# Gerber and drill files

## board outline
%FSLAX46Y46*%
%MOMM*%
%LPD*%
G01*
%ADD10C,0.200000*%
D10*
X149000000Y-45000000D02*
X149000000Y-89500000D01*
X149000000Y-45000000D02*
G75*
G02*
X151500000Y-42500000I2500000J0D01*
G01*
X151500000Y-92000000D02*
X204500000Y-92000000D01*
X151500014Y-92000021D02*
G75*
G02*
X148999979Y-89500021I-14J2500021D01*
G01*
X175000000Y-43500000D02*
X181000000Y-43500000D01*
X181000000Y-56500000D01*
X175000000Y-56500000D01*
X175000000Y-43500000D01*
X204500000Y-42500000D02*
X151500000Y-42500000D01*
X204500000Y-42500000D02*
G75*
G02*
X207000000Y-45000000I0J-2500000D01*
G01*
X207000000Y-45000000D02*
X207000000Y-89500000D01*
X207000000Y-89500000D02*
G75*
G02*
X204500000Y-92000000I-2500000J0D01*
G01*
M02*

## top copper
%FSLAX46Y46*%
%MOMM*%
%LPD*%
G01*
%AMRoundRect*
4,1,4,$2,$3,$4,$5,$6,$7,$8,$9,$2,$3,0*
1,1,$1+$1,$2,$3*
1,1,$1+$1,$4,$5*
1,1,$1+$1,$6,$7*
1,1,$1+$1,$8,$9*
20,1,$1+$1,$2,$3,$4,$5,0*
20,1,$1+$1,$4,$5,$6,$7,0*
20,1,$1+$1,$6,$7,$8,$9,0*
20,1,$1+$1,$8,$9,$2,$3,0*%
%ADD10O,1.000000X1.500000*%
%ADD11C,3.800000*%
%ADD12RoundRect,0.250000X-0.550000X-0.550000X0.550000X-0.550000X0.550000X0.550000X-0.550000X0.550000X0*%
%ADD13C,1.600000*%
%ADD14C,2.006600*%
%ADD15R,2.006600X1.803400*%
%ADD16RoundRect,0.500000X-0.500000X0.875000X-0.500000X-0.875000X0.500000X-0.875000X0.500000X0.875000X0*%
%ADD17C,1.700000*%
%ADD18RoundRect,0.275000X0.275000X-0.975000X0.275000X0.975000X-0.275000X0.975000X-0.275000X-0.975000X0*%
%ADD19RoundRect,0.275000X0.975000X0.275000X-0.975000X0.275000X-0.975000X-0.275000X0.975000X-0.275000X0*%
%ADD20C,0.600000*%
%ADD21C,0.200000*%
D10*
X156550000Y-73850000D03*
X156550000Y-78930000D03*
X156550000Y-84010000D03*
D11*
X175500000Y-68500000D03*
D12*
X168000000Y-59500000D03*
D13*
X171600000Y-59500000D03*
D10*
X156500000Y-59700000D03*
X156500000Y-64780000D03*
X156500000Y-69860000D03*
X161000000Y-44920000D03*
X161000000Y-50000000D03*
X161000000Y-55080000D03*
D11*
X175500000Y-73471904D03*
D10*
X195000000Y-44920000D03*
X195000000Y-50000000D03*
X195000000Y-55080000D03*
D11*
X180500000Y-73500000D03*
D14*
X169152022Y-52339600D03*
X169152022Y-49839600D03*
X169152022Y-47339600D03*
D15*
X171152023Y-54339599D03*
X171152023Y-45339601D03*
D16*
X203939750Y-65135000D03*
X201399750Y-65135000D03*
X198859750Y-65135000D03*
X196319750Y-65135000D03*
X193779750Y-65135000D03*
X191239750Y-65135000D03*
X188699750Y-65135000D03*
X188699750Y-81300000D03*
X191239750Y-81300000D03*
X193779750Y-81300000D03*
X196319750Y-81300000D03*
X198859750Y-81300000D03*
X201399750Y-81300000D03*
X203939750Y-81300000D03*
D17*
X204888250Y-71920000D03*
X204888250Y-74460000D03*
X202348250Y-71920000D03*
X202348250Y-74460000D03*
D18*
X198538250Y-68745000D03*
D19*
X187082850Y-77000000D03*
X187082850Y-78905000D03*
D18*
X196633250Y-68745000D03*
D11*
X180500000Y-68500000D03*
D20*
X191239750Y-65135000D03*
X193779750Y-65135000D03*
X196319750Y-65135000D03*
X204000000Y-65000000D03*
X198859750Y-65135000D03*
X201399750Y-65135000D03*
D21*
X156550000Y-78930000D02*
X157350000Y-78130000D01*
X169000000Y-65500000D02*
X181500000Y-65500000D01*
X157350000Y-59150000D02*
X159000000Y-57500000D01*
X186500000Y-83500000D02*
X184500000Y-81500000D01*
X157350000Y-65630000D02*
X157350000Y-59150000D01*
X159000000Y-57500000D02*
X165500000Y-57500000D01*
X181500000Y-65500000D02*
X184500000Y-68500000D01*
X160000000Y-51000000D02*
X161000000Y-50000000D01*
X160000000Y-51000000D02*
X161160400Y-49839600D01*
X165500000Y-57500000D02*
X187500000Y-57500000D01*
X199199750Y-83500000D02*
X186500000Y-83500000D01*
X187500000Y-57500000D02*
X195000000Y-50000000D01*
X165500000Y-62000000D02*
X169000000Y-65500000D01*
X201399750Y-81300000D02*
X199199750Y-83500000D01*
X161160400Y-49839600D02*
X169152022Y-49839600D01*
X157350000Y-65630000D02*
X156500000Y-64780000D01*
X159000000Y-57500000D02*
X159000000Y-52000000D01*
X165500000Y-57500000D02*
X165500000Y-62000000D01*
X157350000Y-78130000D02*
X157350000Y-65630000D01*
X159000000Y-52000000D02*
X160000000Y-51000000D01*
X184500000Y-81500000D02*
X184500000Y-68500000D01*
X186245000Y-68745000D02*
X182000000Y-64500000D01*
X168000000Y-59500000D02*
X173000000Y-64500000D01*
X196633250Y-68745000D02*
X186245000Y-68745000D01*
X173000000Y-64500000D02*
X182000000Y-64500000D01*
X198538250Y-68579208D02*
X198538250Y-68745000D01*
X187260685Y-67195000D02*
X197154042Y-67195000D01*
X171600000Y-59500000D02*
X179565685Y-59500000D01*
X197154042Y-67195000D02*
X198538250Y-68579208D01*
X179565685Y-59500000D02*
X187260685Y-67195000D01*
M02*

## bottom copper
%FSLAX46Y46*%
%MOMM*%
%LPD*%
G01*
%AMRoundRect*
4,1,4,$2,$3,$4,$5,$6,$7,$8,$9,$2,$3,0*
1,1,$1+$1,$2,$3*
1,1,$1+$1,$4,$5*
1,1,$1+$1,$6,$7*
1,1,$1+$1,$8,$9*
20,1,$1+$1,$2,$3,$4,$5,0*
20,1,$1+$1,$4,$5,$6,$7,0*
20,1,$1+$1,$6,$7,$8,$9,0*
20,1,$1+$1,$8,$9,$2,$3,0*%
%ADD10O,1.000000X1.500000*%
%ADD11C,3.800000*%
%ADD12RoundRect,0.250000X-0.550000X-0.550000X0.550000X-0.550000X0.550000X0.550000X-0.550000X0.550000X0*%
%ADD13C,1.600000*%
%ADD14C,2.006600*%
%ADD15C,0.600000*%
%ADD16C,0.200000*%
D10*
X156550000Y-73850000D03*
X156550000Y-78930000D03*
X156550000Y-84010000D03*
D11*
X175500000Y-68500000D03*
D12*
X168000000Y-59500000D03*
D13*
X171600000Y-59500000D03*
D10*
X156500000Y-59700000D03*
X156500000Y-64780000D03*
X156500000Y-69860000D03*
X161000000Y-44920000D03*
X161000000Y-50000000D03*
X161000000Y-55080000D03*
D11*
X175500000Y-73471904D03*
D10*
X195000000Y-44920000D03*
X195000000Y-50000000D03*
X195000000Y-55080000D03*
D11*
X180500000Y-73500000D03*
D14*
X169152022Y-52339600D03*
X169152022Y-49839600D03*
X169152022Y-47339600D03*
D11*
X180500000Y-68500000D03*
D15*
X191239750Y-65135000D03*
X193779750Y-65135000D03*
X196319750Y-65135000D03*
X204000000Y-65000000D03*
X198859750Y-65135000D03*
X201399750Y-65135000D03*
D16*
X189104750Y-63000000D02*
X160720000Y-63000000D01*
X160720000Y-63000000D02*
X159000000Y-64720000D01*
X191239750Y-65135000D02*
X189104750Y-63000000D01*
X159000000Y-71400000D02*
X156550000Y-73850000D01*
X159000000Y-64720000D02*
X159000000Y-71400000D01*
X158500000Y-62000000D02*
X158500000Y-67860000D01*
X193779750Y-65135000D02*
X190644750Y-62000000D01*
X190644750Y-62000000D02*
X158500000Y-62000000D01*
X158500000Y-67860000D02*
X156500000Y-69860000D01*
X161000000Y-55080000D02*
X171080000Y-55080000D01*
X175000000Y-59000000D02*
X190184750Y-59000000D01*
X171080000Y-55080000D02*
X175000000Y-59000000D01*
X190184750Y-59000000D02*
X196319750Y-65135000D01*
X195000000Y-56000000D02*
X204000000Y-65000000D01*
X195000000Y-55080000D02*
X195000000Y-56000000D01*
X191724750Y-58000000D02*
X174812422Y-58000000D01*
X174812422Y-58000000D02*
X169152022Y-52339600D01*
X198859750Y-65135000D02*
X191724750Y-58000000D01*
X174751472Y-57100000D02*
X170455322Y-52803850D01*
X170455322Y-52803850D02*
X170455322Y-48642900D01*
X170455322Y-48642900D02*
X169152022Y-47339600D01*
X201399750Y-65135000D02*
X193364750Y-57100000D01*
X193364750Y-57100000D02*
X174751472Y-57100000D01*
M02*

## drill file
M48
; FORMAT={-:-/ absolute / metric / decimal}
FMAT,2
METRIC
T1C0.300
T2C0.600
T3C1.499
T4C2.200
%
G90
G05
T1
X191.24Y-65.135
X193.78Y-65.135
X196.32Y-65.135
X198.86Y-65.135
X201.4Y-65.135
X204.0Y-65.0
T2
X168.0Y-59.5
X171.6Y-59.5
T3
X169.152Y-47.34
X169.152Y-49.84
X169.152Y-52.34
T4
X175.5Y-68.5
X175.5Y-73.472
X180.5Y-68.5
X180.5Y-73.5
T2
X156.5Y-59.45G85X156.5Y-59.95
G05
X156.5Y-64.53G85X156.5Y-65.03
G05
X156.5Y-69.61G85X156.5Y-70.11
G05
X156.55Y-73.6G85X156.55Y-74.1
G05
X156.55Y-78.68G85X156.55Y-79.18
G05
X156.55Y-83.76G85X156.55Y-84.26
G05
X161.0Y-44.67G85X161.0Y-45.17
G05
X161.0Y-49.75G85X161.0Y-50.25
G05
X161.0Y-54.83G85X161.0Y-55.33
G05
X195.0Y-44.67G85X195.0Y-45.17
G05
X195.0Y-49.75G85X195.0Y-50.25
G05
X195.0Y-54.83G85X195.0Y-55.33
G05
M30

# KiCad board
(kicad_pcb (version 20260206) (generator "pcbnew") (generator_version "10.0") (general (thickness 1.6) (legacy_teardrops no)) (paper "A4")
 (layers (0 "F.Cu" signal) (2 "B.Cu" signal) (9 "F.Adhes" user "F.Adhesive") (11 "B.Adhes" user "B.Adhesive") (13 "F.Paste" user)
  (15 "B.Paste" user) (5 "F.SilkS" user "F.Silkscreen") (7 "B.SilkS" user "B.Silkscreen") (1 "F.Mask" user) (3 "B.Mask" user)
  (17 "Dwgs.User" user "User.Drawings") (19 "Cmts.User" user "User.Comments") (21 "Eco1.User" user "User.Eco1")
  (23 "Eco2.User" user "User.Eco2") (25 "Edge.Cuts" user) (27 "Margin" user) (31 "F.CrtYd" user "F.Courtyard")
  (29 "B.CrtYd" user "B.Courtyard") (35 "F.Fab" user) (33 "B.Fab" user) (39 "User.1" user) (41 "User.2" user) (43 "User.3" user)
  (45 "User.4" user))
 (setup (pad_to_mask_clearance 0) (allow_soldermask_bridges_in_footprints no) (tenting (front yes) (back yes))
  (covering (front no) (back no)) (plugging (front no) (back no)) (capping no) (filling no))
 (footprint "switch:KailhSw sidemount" (layer "F.Cu") (at 156.55 73.85 -90)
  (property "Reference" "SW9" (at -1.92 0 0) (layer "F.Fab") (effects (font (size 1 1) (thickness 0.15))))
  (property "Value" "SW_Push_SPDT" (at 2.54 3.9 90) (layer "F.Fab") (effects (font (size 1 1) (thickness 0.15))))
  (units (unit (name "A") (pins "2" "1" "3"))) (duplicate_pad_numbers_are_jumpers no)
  (pad "1" thru_hole oval (at 0 0 270) (size 1.5 1) (drill oval 1.1 0.6) (layers "*.Cu" "*.Mask") (remove_unused_layers no) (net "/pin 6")
   (thermal_bridge_angle 45))
  (pad "2" thru_hole oval (at 5.08 0 270) (size 1.5 1) (drill oval 1.1 0.6) (layers "*.Cu" "*.Mask") (remove_unused_layers no)
   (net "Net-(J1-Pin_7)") (thermal_bridge_angle 45))
  (pad "3" thru_hole oval (at 10.16 0 270) (size 1.5 1) (drill oval 1.1 0.6) (layers "*.Cu" "*.Mask") (remove_unused_layers no)
   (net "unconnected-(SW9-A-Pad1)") (thermal_bridge_angle 45)))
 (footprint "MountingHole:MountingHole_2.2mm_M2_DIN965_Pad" (layer "F.Cu") (at 175.5 68.5)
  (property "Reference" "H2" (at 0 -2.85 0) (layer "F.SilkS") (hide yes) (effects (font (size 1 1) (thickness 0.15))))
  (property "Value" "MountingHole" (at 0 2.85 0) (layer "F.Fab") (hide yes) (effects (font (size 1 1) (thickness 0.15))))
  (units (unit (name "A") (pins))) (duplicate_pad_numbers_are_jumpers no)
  (pad "1" thru_hole circle (at 0 0) (size 3.8 3.8) (drill 2.2) (layers "*.Cu" "*.Mask") (remove_unused_layers no) (zone_connect 2)))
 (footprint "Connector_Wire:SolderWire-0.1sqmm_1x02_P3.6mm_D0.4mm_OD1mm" (layer "F.Cu") (at 168 59.5)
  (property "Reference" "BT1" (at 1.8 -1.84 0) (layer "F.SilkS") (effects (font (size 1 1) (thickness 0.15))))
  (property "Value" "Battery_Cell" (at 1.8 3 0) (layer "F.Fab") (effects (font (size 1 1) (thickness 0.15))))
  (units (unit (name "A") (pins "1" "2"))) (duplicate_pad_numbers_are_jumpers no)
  (pad "1" thru_hole roundrect (at 0 0) (size 1.6 1.6) (drill 0.6) (layers "*.Cu" "*.Mask") (remove_unused_layers no)
   (roundrect_rratio 0.15625) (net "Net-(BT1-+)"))
  (pad "2" thru_hole circle (at 3.6 0) (size 1.6 1.6) (drill 0.6) (layers "*.Cu" "*.Mask") (remove_unused_layers no) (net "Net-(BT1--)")))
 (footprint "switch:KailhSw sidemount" (layer "F.Cu") (at 156.5 59.7 -90)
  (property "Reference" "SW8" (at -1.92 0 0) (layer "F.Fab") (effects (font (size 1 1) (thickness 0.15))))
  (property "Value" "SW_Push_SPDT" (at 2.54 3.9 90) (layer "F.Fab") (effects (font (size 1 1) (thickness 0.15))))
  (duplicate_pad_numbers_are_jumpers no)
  (pad "1" thru_hole oval (at 0 0 270) (size 1.5 1) (drill oval 1.1 0.6) (layers "*.Cu" "*.Mask") (remove_unused_layers no)
   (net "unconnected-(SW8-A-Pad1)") (thermal_bridge_angle 45))
  (pad "2" thru_hole oval (at 5.08 0 270) (size 1.5 1) (drill oval 1.1 0.6) (layers "*.Cu" "*.Mask") (remove_unused_layers no)
   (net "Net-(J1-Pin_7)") (thermal_bridge_angle 45))
  (pad "3" thru_hole oval (at 10.16 0 270) (size 1.5 1) (drill oval 1.1 0.6) (layers "*.Cu" "*.Mask") (remove_unused_layers no)
   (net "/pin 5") (thermal_bridge_angle 45)))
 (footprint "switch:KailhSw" (layer "F.Cu") (at 161 44.92 -90)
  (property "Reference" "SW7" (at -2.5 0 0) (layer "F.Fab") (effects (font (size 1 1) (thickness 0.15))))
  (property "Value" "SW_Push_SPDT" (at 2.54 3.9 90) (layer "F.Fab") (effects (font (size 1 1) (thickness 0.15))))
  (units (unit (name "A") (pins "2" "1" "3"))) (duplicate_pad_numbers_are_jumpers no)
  (pad "1" thru_hole oval (at 0 0 270) (size 1.5 1) (drill oval 1.1 0.6) (layers "*.Cu" "*.Mask") (remove_unused_layers no)
   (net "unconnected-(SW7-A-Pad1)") (thermal_bridge_angle 45))
  (pad "2" thru_hole oval (at 5.08 0 270) (size 1.5 1) (drill oval 1.1 0.6) (layers "*.Cu" "*.Mask") (remove_unused_layers no)
   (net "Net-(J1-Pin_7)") (thermal_bridge_angle 45))
  (pad "3" thru_hole oval (at 10.16 0 270) (size 1.5 1) (drill oval 1.1 0.6) (layers "*.Cu" "*.Mask") (remove_unused_layers no)
   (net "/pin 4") (thermal_bridge_angle 45)))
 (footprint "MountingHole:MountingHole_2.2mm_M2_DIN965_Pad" (layer "F.Cu") (at 175.5 73.471904)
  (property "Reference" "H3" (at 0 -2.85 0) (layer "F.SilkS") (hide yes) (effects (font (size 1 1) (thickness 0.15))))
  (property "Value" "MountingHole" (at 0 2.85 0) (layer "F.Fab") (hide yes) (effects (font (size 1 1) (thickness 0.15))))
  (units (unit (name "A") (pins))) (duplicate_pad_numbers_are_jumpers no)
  (pad "1" thru_hole circle (at 0 0) (size 3.8 3.8) (drill 2.2) (layers "*.Cu" "*.Mask") (remove_unused_layers no) (zone_connect 2)))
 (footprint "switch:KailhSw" (layer "F.Cu") (at 195 44.92 -90)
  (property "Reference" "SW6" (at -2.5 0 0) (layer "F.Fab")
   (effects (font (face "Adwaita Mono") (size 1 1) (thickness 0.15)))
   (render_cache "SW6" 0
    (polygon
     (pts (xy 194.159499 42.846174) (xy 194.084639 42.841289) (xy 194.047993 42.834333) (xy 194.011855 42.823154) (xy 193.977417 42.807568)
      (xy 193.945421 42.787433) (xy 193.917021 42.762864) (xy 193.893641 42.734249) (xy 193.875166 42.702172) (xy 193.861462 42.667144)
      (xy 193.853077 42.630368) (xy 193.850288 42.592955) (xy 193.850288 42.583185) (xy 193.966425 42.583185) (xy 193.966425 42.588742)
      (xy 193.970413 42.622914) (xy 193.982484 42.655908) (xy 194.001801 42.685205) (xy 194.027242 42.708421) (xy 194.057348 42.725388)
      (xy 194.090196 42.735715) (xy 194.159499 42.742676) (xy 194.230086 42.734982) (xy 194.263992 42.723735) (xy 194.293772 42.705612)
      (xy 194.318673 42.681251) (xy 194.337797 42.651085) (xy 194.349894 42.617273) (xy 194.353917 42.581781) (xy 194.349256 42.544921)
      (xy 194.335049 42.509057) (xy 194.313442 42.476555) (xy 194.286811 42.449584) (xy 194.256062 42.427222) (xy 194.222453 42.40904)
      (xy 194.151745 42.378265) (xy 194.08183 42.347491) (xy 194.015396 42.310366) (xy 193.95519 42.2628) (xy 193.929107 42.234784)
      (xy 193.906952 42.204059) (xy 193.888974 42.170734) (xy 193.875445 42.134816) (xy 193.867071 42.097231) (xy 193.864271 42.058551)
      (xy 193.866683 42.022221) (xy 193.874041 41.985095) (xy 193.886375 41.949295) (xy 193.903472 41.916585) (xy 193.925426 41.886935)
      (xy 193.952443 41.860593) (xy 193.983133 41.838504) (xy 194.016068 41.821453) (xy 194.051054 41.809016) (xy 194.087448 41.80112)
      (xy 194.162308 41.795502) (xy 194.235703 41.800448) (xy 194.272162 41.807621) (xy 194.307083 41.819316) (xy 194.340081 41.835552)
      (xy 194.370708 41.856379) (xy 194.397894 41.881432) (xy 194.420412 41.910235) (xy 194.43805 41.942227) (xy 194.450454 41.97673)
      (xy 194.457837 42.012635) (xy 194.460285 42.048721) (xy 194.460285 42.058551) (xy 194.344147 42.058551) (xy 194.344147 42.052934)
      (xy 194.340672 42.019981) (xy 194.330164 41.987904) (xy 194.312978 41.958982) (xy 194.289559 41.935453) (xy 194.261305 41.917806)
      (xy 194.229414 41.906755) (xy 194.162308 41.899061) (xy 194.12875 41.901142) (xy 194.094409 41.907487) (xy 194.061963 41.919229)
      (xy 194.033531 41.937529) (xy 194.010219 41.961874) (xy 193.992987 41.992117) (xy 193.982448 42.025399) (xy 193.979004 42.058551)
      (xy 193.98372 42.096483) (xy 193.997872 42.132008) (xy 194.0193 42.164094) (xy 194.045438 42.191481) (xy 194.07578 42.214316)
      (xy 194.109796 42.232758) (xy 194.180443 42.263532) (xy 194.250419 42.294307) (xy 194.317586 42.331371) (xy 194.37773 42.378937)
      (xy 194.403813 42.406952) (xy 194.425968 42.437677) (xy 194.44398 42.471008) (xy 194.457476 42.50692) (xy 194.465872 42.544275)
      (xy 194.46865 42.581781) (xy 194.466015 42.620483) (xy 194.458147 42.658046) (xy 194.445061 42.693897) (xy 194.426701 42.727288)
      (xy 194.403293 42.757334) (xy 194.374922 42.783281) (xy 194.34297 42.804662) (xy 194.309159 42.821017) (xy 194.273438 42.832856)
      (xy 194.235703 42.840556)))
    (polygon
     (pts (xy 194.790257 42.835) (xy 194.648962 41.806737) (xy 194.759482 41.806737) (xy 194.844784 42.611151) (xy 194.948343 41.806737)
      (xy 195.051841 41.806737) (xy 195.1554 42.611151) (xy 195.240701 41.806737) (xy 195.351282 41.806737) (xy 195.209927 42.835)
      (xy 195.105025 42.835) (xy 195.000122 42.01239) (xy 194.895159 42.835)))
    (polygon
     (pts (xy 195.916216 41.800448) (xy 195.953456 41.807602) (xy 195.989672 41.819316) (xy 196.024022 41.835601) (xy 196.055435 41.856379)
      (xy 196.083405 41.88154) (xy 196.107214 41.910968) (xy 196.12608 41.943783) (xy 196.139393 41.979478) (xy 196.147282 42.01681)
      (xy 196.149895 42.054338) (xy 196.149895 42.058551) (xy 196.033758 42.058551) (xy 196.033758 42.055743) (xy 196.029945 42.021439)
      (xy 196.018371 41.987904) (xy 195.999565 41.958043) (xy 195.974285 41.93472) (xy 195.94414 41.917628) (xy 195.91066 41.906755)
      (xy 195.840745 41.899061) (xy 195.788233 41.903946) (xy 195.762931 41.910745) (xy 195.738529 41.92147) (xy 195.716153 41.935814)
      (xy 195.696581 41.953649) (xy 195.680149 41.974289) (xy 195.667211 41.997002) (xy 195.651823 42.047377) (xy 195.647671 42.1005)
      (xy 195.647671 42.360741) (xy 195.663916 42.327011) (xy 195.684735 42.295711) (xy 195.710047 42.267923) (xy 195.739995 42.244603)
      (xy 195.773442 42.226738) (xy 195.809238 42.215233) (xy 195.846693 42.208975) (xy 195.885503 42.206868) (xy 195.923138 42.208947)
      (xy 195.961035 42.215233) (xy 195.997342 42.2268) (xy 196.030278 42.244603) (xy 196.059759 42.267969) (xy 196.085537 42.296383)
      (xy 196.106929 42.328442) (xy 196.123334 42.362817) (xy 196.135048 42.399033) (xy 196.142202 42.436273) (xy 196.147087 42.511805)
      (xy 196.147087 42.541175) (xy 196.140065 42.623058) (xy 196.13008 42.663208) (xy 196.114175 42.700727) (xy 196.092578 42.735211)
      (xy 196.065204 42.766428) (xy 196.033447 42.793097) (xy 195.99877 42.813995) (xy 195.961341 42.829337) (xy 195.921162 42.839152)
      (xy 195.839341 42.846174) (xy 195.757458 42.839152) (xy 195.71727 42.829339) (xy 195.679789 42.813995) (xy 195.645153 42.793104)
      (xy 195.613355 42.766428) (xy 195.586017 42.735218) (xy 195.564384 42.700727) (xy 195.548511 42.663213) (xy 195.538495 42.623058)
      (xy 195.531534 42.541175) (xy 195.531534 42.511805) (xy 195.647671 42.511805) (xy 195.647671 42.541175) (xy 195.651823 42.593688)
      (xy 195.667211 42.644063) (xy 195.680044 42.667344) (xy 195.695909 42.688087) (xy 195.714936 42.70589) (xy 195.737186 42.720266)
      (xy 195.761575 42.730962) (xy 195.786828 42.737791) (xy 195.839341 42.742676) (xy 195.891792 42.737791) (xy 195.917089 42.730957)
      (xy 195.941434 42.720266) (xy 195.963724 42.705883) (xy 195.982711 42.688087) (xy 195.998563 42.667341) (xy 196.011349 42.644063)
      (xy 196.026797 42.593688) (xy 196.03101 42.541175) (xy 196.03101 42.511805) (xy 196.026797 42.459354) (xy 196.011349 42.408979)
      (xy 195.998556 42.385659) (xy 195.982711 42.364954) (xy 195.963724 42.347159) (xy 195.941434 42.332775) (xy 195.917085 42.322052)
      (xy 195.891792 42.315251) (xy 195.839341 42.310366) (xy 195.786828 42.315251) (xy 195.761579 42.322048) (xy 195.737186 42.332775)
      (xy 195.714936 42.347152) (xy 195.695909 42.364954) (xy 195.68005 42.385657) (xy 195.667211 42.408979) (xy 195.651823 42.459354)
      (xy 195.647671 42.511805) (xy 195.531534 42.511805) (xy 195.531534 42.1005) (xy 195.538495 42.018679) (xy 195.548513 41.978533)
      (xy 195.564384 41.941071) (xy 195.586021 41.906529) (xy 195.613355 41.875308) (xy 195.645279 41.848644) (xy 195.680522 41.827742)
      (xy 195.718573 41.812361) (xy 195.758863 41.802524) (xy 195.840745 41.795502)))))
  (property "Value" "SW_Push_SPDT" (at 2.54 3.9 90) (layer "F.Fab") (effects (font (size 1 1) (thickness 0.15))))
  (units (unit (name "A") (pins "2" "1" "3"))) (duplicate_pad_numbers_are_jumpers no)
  (pad "1" thru_hole oval (at 0 0 270) (size 1.5 1) (drill oval 1.1 0.6) (layers "*.Cu" "*.Mask") (remove_unused_layers no)
   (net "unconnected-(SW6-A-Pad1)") (thermal_bridge_angle 45))
  (pad "2" thru_hole oval (at 5.08 0 270) (size 1.5 1) (drill oval 1.1 0.6) (layers "*.Cu" "*.Mask") (remove_unused_layers no)
   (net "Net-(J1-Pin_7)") (thermal_bridge_angle 45))
  (pad "3" thru_hole oval (at 10.16 0 270) (size 1.5 1) (drill oval 1.1 0.6) (layers "*.Cu" "*.Mask") (remove_unused_layers no)
   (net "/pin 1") (thermal_bridge_angle 45)))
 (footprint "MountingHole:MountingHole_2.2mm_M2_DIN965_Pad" (layer "F.Cu") (at 180.5 73.5)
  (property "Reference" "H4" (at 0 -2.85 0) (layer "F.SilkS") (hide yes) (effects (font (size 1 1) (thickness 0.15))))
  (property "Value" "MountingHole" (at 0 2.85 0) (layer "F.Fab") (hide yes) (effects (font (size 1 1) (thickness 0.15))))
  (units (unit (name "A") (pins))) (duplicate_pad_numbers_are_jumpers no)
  (pad "1" thru_hole circle (at 0 0) (size 3.8 3.8) (drill 2.2) (layers "*.Cu" "*.Mask") (remove_unused_layers no) (zone_connect 2)))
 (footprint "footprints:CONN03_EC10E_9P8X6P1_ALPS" (layer "F.Cu") (at 169.152022 52.3396 90)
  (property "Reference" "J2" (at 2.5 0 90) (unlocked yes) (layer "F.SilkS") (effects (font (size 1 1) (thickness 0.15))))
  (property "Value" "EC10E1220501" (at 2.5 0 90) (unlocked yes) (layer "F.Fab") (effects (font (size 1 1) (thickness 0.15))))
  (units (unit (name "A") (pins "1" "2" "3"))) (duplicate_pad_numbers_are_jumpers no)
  (pad "1" thru_hole circle (at 0 0 90) (size 2.0066 2.0066) (drill 1.4986) (layers "*.Cu" "*.Mask") (remove_unused_layers no)
   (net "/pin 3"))
  (pad "2" thru_hole circle (at 2.5 0 90) (size 2.0066 2.0066) (drill 1.4986) (layers "*.Cu" "*.Mask") (remove_unused_layers no)
   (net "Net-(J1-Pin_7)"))
  (pad "3" thru_hole circle (at 5 0 90) (size 2.0066 2.0066) (drill 1.4986) (layers "*.Cu" "*.Mask") (remove_unused_layers no)
   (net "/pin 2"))
  (pad "4" smd rect (at -1.999999 2.000001 90) (size 1.8034 2.0066) (layers "F.Cu" "F.Mask" "F.Paste"))
  (pad "5" smd rect (at 6.999999 2.000001 90) (size 1.8034 2.0066) (layers "F.Cu" "F.Mask" "F.Paste")))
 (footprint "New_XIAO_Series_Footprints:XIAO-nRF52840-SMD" (layer "F.Cu") (at 185.81975 64.3 -90)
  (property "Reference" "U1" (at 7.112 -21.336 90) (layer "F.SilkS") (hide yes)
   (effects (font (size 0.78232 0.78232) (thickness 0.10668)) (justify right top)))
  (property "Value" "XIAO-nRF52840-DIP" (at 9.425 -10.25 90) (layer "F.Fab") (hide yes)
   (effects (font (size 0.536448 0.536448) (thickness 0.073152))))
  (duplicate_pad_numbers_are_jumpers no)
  (pad "1" smd roundrect (at 0.835 -18.12 270) (size 2.75 2) (layers "F.Cu" "F.Mask" "F.Paste") (roundrect_rratio 0.25) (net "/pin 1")
   (solder_mask_margin 0.0508) (thermal_bridge_angle 45))
  (pad "2" smd roundrect (at 0.835 -15.58 270) (size 2.75 2) (layers "F.Cu" "F.Mask" "F.Paste") (roundrect_rratio 0.25) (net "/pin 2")
   (solder_mask_margin 0.0508) (thermal_bridge_angle 45))
  (pad "3" smd roundrect (at 0.835 -13.04 270) (size 2.75 2) (layers "F.Cu" "F.Mask" "F.Paste") (roundrect_rratio 0.25) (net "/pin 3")
   (solder_mask_margin 0.0508) (thermal_bridge_angle 45))
  (pad "4" smd roundrect (at 0.835 -10.5 270) (size 2.75 2) (layers "F.Cu" "F.Mask" "F.Paste") (roundrect_rratio 0.25) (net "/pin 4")
   (solder_mask_margin 0.0508) (thermal_bridge_angle 45))
  (pad "5" smd roundrect (at 0.835 -7.96 270) (size 2.75 2) (layers "F.Cu" "F.Mask" "F.Paste") (roundrect_rratio 0.25) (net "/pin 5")
   (solder_mask_margin 0.0508) (thermal_bridge_angle 45))
  (pad "6" smd roundrect (at 0.835 -5.42 270) (size 2.75 2) (layers "F.Cu" "F.Mask" "F.Paste") (roundrect_rratio 0.25) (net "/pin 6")
   (solder_mask_margin 0.0508) (thermal_bridge_angle 45))
  (pad "7" smd roundrect (at 0.835 -2.88 270) (size 2.75 2) (layers "F.Cu" "F.Mask" "F.Paste") (roundrect_rratio 0.25)
   (solder_mask_margin 0.0508) (thermal_bridge_angle 45))
  (pad "8" smd roundrect (at 17 -2.88 270) (size 2.75 2) (layers "F.Cu" "F.Mask" "F.Paste") (roundrect_rratio 0.25) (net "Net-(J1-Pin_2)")
   (solder_mask_margin 0.0508) (thermal_bridge_angle 45))
  (pad "9" smd roundrect (at 17 -5.42 270) (size 2.75 2) (layers "F.Cu" "F.Mask" "F.Paste") (roundrect_rratio 0.25) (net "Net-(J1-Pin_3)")
   (solder_mask_margin 0.0508) (thermal_bridge_angle 45))
  (pad "10" smd roundrect (at 17 -7.96 270) (size 2.75 2) (layers "F.Cu" "F.Mask" "F.Paste") (roundrect_rratio 0.25) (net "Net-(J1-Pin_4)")
   (solder_mask_margin 0.0508) (thermal_bridge_angle 45))
  (pad "11" smd roundrect (at 17 -10.5 270) (size 2.75 2) (layers "F.Cu" "F.Mask" "F.Paste") (roundrect_rratio 0.25) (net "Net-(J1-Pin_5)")
   (solder_mask_margin 0.0508) (thermal_bridge_angle 45))
  (pad "12" smd roundrect (at 17 -13.04 270) (size 2.75 2) (layers "F.Cu" "F.Mask" "F.Paste") (roundrect_rratio 0.25) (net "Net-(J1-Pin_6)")
   (solder_mask_margin 0.0508) (thermal_bridge_angle 45))
  (pad "13" smd roundrect (at 17 -15.58 270) (size 2.75 2) (layers "F.Cu" "F.Mask" "F.Paste") (roundrect_rratio 0.25) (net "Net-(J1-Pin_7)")
   (solder_mask_margin 0.0508) (thermal_bridge_angle 45))
  (pad "14" smd roundrect (at 17 -18.12 270) (size 2.75 2) (layers "F.Cu" "F.Mask" "F.Paste") (roundrect_rratio 0.25)
   (solder_mask_margin 0.0508) (thermal_bridge_angle 45))
  (pad "15" smd circle (at 7.62 -19.0685 270) (size 1.7 1.7) (layers "F.Cu" "F.Mask" "F.Paste"))
  (pad "16" smd circle (at 10.16 -19.0685 270) (size 1.7 1.7) (layers "F.Cu" "F.Mask" "F.Paste"))
  (pad "17" smd circle (at 7.62 -16.5285 270) (size 1.7 1.7) (layers "F.Cu" "F.Mask" "F.Paste"))
  (pad "18" smd circle (at 10.16 -16.5285 270) (size 1.7 1.7) (layers "F.Cu" "F.Mask" "F.Paste"))
  (pad "20" smd roundrect (at 4.445 -12.7185 90) (size 2.5 1.1) (layers "F.Cu" "F.Mask" "F.Paste") (roundrect_rratio 0.25)
   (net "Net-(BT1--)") (thermal_bridge_angle 45))
  (pad "21" smd roundrect (at 12.7 -1.2631 180) (size 2.5 1.1) (layers "F.Cu" "F.Mask" "F.Paste") (roundrect_rratio 0.25)
   (thermal_bridge_angle 45))
  (pad "22" smd roundrect (at 14.605 -1.2631 180) (size 2.5 1.1) (layers "F.Cu" "F.Mask" "F.Paste") (roundrect_rratio 0.25)
   (thermal_bridge_angle 45))
  (pad "hy" smd roundrect (at 4.445 -10.8135 90) (size 2.5 1.1) (layers "F.Cu" "F.Mask" "F.Paste") (roundrect_rratio 0.25)
   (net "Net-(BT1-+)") (thermal_bridge_angle 45)))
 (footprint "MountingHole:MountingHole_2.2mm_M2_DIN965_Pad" (layer "F.Cu") (at 180.5 68.5)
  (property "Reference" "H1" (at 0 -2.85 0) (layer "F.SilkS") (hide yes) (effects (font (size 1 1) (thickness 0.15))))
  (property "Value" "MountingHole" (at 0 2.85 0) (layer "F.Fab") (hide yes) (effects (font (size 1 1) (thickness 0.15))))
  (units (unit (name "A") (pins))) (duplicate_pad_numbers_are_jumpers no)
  (pad "1" thru_hole circle (at 0 0) (size 3.8 3.8) (drill 2.2) (layers "*.Cu" "*.Mask") (remove_unused_layers no) (zone_connect 2)))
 (gr_line (start 149 45) (end 149 89.5) (stroke (width 0.2) (type solid)) (layer "Edge.Cuts"))
 (gr_arc (start 149 45) (mid 149.732233 43.232233) (end 151.5 42.5) (stroke (width 0.2) (type solid)) (layer "Edge.Cuts"))
 (gr_line (start 151.5 92) (end 204.5 92) (stroke (width 0.2) (type solid)) (layer "Edge.Cuts"))
 (gr_arc (start 151.500014 92.000021) (mid 149.732266 91.267788) (end 149.000014 89.500021) (stroke (width 0.2) (type solid))
  (layer "Edge.Cuts"))
 (gr_rect (start 175 43.5) (end 181 56.5) (stroke (width 0.2) (type solid)) (fill no) (layer "Edge.Cuts"))
 (gr_line (start 204.5 42.5) (end 151.5 42.5) (stroke (width 0.2) (type solid)) (layer "Edge.Cuts"))
 (gr_arc (start 204.5 42.5) (mid 206.267767 43.232233) (end 207 45) (stroke (width 0.2) (type solid)) (layer "Edge.Cuts"))
 (gr_line (start 207 45) (end 207 89.5) (stroke (width 0.2) (type solid)) (layer "Edge.Cuts"))
 (gr_arc (start 207 89.5) (mid 206.267767 91.267767) (end 204.5 92) (stroke (width 0.2) (type solid)) (layer "Edge.Cuts"))
 (segment (start 156.55 78.93) (end 157.35 78.13) (width 0.2) (layer "F.Cu") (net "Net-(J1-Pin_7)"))
 (segment (start 169 65.5) (end 181.5 65.5) (width 0.2) (layer "F.Cu") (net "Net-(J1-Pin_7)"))
 (segment (start 157.35 59.15) (end 159 57.5) (width 0.2) (layer "F.Cu") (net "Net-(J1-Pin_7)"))
 (segment (start 186.5 83.5) (end 184.5 81.5) (width 0.2) (layer "F.Cu") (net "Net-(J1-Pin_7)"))
 (segment (start 157.35 65.63) (end 157.35 59.15) (width 0.2) (layer "F.Cu") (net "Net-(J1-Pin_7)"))
 (segment (start 159 57.5) (end 165.5 57.5) (width 0.2) (layer "F.Cu") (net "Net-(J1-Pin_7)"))
 (segment (start 181.5 65.5) (end 184.5 68.5) (width 0.2) (layer "F.Cu") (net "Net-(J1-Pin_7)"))
 (segment (start 160 51) (end 161 50) (width 0.2) (layer "F.Cu") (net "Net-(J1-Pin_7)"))
 (segment (start 160 51) (end 161.1604 49.8396) (width 0.2) (layer "F.Cu") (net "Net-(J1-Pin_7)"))
 (segment (start 165.5 57.5) (end 187.5 57.5) (width 0.2) (layer "F.Cu") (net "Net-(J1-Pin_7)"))
 (segment (start 199.19975 83.5) (end 186.5 83.5) (width 0.2) (layer "F.Cu") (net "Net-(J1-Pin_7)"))
 (segment (start 187.5 57.5) (end 195 50) (width 0.2) (layer "F.Cu") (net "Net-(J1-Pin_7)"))
 (segment (start 165.5 62) (end 169 65.5) (width 0.2) (layer "F.Cu") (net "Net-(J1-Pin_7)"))
 (segment (start 201.39975 81.3) (end 199.19975 83.5) (width 0.2) (layer "F.Cu") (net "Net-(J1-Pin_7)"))
 (segment (start 161.1604 49.8396) (end 169.152022 49.8396) (width 0.2) (layer "F.Cu") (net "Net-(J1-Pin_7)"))
 (segment (start 157.35 65.63) (end 156.5 64.78) (width 0.2) (layer "F.Cu") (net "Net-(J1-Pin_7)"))
 (segment (start 159 57.5) (end 159 52) (width 0.2) (layer "F.Cu") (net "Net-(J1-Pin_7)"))
 (segment (start 165.5 57.5) (end 165.5 62) (width 0.2) (layer "F.Cu") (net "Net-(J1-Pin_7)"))
 (segment (start 157.35 78.13) (end 157.35 65.63) (width 0.2) (layer "F.Cu") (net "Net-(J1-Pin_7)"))
 (segment (start 159 52) (end 160 51) (width 0.2) (layer "F.Cu") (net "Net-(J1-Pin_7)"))
 (segment (start 184.5 81.5) (end 184.5 68.5) (width 0.2) (layer "F.Cu") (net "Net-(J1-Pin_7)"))
 (via (at 191.23975 65.135) (size 0.6) (drill 0.3) (layers "F.Cu" "B.Cu") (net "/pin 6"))
 (segment (start 189.10475 63) (end 160.72 63) (width 0.2) (layer "B.Cu") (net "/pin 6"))
 (segment (start 160.72 63) (end 159 64.72) (width 0.2) (layer "B.Cu") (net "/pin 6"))
 (segment (start 191.23975 65.135) (end 189.10475 63) (width 0.2) (layer "B.Cu") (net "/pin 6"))
 (segment (start 159 71.4) (end 156.55 73.85) (width 0.2) (layer "B.Cu") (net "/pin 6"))
 (segment (start 159 64.72) (end 159 71.4) (width 0.2) (layer "B.Cu") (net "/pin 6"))
 (segment (start 186.245 68.745) (end 182 64.5) (width 0.2) (layer "F.Cu") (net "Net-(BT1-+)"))
 (segment (start 168 59.5) (end 173 64.5) (width 0.2) (layer "F.Cu") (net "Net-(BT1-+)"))
 (segment (start 196.63325 68.745) (end 186.245 68.745) (width 0.2) (layer "F.Cu") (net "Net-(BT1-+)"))
 (segment (start 173 64.5) (end 182 64.5) (width 0.2) (layer "F.Cu") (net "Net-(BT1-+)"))
 (segment (start 198.53825 68.579208) (end 198.53825 68.745) (width 0.2) (layer "F.Cu") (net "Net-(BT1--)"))
 (segment (start 187.260685 67.195) (end 197.154042 67.195) (width 0.2) (layer "F.Cu") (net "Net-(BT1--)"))
 (segment (start 171.6 59.5) (end 179.565685 59.5) (width 0.2) (layer "F.Cu") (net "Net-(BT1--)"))
 (segment (start 197.154042 67.195) (end 198.53825 68.579208) (width 0.2) (layer "F.Cu") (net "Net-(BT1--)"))
 (segment (start 179.565685 59.5) (end 187.260685 67.195) (width 0.2) (layer "F.Cu") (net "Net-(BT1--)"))
 (via (at 193.77975 65.135) (size 0.6) (drill 0.3) (layers "F.Cu" "B.Cu") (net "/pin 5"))
 (segment (start 158.5 62) (end 158.5 67.86) (width 0.2) (layer "B.Cu") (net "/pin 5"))
 (segment (start 193.77975 65.135) (end 190.64475 62) (width 0.2) (layer "B.Cu") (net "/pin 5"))
 (segment (start 190.64475 62) (end 158.5 62) (width 0.2) (layer "B.Cu") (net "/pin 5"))
 (segment (start 158.5 67.86) (end 156.5 69.86) (width 0.2) (layer "B.Cu") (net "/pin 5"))
 (via (at 196.31975 65.135) (size 0.6) (drill 0.3) (layers "F.Cu" "B.Cu") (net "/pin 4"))
 (segment (start 161 55.08) (end 171.08 55.08) (width 0.2) (layer "B.Cu") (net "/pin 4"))
 (segment (start 175 59) (end 190.18475 59) (width 0.2) (layer "B.Cu") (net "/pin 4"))
 (segment (start 171.08 55.08) (end 175 59) (width 0.2) (layer "B.Cu") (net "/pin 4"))
 (segment (start 190.18475 59) (end 196.31975 65.135) (width 0.2) (layer "B.Cu") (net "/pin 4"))
 (via (at 204 65) (size 0.6) (drill 0.3) (layers "F.Cu" "B.Cu") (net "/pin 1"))
 (segment (start 195 56) (end 204 65) (width 0.2) (layer "B.Cu") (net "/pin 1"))
 (segment (start 195 55.08) (end 195 56) (width 0.2) (layer "B.Cu") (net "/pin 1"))
 (via (at 198.85975 65.135) (size 0.6) (drill 0.3) (layers "F.Cu" "B.Cu") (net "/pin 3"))
 (segment (start 191.72475 58) (end 174.812422 58) (width 0.2) (layer "B.Cu") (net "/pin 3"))
 (segment (start 174.812422 58) (end 169.152022 52.3396) (width 0.2) (layer "B.Cu") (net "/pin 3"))
 (segment (start 198.85975 65.135) (end 191.72475 58) (width 0.2) (layer "B.Cu") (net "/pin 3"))
 (via (at 201.39975 65.135) (size 0.6) (drill 0.3) (layers "F.Cu" "B.Cu") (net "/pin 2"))
 (segment (start 174.751472 57.1) (end 170.455322 52.80385) (width 0.2) (layer "B.Cu") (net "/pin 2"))
 (segment (start 170.455322 52.80385) (end 170.455322 48.6429) (width 0.2) (layer "B.Cu") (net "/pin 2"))
 (segment (start 170.455322 48.6429) (end 169.152022 47.3396) (width 0.2) (layer "B.Cu") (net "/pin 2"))
 (segment (start 201.39975 65.135) (end 193.36475 57.1) (width 0.2) (layer "B.Cu") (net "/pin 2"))
 (segment (start 193.36475 57.1) (end 174.751472 57.1) (width 0.2) (layer "B.Cu") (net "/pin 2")))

